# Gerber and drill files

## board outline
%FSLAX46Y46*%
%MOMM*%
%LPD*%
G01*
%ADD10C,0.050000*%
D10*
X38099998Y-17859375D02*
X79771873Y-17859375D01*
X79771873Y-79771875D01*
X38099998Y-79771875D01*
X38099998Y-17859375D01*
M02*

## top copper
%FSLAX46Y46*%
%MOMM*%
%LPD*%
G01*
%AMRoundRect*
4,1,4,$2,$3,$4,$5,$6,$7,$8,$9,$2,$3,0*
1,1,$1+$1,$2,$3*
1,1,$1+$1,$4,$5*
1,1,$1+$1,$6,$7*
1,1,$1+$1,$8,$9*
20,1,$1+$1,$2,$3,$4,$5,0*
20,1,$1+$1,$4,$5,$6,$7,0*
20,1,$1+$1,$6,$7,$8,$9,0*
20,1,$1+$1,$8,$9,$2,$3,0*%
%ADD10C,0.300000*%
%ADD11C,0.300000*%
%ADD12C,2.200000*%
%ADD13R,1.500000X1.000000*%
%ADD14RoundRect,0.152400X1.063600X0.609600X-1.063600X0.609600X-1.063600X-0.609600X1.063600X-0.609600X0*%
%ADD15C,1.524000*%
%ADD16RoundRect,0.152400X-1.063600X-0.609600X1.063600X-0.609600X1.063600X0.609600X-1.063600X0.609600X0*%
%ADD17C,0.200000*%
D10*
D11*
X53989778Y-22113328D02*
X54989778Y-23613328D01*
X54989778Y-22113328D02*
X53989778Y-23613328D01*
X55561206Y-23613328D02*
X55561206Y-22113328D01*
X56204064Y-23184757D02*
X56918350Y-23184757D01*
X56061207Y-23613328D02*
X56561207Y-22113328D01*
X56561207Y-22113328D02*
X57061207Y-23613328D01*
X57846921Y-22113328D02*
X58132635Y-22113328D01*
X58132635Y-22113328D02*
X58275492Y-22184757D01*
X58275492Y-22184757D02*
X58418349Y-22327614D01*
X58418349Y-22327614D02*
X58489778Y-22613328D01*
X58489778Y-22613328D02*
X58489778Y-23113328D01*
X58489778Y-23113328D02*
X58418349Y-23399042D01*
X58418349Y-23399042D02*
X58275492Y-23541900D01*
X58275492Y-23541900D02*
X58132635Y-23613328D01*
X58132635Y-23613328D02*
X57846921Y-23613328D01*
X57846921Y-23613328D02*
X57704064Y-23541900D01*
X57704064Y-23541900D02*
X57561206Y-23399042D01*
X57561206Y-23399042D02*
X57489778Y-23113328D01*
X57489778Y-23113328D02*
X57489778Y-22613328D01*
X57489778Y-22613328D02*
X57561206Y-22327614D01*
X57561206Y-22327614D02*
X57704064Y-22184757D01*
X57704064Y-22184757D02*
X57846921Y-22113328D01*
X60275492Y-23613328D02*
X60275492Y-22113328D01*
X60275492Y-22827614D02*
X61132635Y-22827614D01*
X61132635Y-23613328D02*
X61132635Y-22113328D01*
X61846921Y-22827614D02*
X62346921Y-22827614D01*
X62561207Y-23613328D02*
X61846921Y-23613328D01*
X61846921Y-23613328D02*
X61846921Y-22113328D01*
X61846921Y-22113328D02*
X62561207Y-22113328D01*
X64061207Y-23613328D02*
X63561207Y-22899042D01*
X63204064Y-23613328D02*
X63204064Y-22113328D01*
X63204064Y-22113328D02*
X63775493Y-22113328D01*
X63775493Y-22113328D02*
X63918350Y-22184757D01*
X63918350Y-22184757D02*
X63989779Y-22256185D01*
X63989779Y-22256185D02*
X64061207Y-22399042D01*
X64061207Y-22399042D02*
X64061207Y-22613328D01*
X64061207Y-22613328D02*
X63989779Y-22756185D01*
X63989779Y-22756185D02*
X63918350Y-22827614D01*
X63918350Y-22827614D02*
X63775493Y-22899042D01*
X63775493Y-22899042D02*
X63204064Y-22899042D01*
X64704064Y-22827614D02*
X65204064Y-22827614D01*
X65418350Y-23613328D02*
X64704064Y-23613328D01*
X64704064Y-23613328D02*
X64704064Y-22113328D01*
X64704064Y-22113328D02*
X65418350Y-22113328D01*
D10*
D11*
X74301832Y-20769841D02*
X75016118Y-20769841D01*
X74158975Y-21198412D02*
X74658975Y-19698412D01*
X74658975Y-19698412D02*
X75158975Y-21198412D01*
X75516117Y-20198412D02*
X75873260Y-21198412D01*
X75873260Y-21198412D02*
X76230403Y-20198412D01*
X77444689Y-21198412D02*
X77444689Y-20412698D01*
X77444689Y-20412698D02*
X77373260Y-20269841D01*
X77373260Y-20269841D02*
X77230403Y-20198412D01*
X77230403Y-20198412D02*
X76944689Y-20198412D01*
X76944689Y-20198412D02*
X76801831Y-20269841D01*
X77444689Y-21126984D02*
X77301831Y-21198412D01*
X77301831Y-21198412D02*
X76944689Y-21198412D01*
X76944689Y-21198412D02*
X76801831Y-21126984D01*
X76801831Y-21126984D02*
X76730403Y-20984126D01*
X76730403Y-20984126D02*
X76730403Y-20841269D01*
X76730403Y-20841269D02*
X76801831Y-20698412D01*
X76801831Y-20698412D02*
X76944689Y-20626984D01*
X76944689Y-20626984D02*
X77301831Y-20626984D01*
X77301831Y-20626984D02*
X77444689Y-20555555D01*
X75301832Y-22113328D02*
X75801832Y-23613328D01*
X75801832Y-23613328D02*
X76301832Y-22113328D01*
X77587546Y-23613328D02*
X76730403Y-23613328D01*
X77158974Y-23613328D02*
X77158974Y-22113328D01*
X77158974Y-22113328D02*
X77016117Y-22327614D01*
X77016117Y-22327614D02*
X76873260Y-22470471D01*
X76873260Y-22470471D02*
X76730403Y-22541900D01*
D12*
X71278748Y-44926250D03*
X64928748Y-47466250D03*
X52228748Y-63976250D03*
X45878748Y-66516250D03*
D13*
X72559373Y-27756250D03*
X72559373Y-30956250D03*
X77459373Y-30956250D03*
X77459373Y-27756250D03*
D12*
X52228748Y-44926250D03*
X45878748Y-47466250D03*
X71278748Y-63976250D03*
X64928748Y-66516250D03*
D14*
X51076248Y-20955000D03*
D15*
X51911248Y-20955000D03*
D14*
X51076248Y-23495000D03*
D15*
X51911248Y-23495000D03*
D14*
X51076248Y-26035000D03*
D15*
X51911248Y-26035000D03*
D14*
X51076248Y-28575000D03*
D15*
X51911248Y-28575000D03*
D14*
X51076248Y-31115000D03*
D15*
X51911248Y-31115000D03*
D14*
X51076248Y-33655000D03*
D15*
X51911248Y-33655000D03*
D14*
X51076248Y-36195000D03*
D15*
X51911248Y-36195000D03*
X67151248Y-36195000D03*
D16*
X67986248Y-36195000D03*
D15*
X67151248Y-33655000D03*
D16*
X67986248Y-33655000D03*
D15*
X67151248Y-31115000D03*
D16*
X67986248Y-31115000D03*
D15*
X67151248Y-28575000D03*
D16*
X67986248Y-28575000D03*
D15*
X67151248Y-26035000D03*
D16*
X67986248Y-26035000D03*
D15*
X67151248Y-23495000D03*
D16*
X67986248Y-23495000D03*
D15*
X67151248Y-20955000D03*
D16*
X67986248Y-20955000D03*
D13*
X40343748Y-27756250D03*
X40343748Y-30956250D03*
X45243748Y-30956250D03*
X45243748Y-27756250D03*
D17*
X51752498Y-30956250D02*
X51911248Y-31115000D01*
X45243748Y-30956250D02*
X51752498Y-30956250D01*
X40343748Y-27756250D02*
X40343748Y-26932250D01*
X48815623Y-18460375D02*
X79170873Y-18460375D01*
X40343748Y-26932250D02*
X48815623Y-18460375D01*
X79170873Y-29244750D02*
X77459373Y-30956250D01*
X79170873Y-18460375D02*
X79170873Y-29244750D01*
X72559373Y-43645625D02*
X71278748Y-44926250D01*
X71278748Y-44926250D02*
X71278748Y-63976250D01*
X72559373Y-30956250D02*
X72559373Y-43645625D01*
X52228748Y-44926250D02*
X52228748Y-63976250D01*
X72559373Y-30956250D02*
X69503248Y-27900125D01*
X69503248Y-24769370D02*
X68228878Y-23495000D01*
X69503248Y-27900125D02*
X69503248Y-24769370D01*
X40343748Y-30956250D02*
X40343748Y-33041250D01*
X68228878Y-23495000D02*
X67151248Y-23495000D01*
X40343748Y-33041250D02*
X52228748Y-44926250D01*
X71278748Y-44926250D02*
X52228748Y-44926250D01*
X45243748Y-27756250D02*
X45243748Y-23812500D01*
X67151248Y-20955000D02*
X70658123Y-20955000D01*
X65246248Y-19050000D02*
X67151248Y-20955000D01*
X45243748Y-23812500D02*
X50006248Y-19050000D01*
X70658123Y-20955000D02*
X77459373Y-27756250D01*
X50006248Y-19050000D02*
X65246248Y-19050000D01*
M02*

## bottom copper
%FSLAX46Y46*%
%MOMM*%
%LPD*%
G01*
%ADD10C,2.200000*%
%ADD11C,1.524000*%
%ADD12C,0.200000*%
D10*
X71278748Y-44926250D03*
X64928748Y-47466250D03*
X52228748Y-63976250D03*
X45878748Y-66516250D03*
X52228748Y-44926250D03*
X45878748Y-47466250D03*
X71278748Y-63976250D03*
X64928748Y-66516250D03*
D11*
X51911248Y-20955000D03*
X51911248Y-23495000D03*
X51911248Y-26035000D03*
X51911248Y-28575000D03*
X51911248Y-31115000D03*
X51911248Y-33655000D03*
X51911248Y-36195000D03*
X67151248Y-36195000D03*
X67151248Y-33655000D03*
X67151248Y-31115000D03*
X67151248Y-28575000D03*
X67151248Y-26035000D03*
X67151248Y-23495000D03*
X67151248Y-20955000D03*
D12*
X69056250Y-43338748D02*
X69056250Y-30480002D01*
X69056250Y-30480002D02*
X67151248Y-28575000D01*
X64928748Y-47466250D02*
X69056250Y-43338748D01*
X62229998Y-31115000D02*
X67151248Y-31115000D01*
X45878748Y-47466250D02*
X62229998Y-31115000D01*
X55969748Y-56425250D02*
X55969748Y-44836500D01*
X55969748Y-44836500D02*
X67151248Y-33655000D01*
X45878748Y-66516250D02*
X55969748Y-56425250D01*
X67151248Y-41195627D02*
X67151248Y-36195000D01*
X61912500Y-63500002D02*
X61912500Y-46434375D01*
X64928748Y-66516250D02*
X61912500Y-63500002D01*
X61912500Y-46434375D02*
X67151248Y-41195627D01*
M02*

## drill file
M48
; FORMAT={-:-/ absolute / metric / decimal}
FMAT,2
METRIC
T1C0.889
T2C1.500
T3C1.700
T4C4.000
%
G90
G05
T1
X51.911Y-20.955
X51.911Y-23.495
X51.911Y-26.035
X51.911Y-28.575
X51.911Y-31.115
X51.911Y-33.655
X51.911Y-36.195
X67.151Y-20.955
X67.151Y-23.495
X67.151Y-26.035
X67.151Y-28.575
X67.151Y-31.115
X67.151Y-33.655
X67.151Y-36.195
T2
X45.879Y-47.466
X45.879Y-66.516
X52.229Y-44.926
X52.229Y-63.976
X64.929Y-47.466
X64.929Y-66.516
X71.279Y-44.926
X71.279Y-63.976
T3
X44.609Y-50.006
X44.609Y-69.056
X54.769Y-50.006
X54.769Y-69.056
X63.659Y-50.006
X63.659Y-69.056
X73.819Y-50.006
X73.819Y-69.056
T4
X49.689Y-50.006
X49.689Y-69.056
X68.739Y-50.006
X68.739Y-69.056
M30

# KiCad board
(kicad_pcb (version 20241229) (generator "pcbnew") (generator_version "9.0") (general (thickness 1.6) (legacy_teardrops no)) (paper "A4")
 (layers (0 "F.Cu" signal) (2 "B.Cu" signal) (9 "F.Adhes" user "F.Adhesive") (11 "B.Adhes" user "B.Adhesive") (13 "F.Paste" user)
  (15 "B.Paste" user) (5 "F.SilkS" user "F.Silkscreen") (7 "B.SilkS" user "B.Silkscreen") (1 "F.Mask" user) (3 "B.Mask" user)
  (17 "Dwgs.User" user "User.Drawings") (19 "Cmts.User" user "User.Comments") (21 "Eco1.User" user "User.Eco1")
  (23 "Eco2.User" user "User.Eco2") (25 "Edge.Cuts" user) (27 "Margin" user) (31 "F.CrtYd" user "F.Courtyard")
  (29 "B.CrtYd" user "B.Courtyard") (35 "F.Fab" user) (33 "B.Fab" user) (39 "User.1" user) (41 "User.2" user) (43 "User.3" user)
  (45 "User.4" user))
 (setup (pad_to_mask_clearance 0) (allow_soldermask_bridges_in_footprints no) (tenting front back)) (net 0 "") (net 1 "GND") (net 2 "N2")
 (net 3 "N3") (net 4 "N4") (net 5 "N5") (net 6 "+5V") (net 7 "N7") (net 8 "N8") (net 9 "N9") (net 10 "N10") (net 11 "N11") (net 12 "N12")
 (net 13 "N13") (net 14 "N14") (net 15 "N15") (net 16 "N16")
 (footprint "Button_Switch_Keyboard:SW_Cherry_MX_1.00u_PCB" (layer "F.Cu") (at 71.278748 44.92625)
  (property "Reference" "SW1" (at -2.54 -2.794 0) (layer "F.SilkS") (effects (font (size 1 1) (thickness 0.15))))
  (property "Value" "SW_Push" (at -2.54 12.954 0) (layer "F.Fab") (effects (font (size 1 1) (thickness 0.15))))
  (pad "" np_thru_hole circle (at -7.62 5.08) (size 1.7 1.7) (drill 1.7) (layers "*.Cu" "*.Mask"))
  (pad "" np_thru_hole circle (at -2.54 5.08) (size 4 4) (drill 4) (layers "*.Cu" "*.Mask"))
  (pad "" np_thru_hole circle (at 2.54 5.08) (size 1.7 1.7) (drill 1.7) (layers "*.Cu" "*.Mask"))
  (pad "1" thru_hole circle (at 0 0) (size 2.2 2.2) (drill 1.5) (layers "*.Cu" "*.Mask") (remove_unused_layers no) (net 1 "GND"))
  (pad "2" thru_hole circle (at -6.35 2.54) (size 2.2 2.2) (drill 1.5) (layers "*.Cu" "*.Mask") (remove_unused_layers no) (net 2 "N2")))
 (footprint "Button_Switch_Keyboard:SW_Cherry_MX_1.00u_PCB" (layer "F.Cu") (at 52.228748 63.97625)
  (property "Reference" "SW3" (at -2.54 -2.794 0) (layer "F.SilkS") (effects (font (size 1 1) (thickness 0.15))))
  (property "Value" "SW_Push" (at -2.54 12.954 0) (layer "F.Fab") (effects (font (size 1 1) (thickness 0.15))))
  (pad "" np_thru_hole circle (at -7.62 5.08) (size 1.7 1.7) (drill 1.7) (layers "*.Cu" "*.Mask"))
  (pad "" np_thru_hole circle (at -2.54 5.08) (size 4 4) (drill 4) (layers "*.Cu" "*.Mask"))
  (pad "" np_thru_hole circle (at 2.54 5.08) (size 1.7 1.7) (drill 1.7) (layers "*.Cu" "*.Mask"))
  (pad "1" thru_hole circle (at 0 0) (size 2.2 2.2) (drill 1.5) (layers "*.Cu" "*.Mask") (remove_unused_layers no) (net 1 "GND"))
  (pad "2" thru_hole circle (at -6.35 2.54) (size 2.2 2.2) (drill 1.5) (layers "*.Cu" "*.Mask") (remove_unused_layers no) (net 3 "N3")))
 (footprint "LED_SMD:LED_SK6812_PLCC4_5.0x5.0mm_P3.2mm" (layer "F.Cu") (at 75.009373 29.35625)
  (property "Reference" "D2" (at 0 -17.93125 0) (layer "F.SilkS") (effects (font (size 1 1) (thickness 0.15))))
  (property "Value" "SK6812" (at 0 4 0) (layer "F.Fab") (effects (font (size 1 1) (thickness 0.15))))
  (pad "1" smd rect (at -2.45 -1.6 180) (size 1.5 1) (layers "F.Cu" "F.Mask" "F.Paste") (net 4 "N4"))
  (pad "2" smd rect (at -2.45 1.6 180) (size 1.5 1) (layers "F.Cu" "F.Mask" "F.Paste") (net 1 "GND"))
  (pad "3" smd rect (at 2.45 1.6 180) (size 1.5 1) (layers "F.Cu" "F.Mask" "F.Paste") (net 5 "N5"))
  (pad "4" smd rect (at 2.45 -1.6 180) (size 1.5 1) (layers "F.Cu" "F.Mask" "F.Paste") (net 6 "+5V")))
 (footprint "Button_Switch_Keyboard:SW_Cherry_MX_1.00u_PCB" (layer "F.Cu") (at 52.228748 44.92625)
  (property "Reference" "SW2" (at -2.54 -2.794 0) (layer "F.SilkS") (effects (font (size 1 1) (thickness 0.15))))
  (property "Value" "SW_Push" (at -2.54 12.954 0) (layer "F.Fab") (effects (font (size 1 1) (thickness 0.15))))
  (pad "" np_thru_hole circle (at -7.62 5.08) (size 1.7 1.7) (drill 1.7) (layers "*.Cu" "*.Mask"))
  (pad "" np_thru_hole circle (at -2.54 5.08) (size 4 4) (drill 4) (layers "*.Cu" "*.Mask"))
  (pad "" np_thru_hole circle (at 2.54 5.08) (size 1.7 1.7) (drill 1.7) (layers "*.Cu" "*.Mask"))
  (pad "1" thru_hole circle (at 0 0) (size 2.2 2.2) (drill 1.5) (layers "*.Cu" "*.Mask") (remove_unused_layers no) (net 1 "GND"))
  (pad "2" thru_hole circle (at -6.35 2.54) (size 2.2 2.2) (drill 1.5) (layers "*.Cu" "*.Mask") (remove_unused_layers no) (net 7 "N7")))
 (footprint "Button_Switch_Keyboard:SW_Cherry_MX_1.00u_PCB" (layer "F.Cu") (at 71.278748 63.97625)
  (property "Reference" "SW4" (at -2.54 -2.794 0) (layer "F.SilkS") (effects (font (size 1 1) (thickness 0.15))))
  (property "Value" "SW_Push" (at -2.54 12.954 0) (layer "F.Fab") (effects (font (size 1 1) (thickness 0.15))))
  (pad "" np_thru_hole circle (at -7.62 5.08) (size 1.7 1.7) (drill 1.7) (layers "*.Cu" "*.Mask"))
  (pad "" np_thru_hole circle (at -2.54 5.08) (size 4 4) (drill 4) (layers "*.Cu" "*.Mask"))
  (pad "" np_thru_hole circle (at 2.54 5.08) (size 1.7 1.7) (drill 1.7) (layers "*.Cu" "*.Mask"))
  (pad "1" thru_hole circle (at 0 0) (size 2.2 2.2) (drill 1.5) (layers "*.Cu" "*.Mask") (remove_unused_layers no) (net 1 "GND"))
  (pad "2" thru_hole circle (at -6.35 2.54) (size 2.2 2.2) (drill 1.5) (layers "*.Cu" "*.Mask") (remove_unused_layers no) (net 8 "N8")))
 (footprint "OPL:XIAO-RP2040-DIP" (layer "F.Cu") (at 59.531248 28.575)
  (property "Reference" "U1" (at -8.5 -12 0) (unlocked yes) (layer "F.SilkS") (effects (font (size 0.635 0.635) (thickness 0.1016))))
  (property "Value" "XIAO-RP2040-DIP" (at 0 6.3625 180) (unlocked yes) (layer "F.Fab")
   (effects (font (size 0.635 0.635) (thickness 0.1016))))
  (pad "1" smd roundrect (at -8.455 -7.62 180) (size 2.432 1.524) (layers "F.Cu" "F.Mask") (roundrect_rratio 0.1) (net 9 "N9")
   (thermal_bridge_angle 45))
  (pad "1" thru_hole circle (at -7.62 -7.62 180) (size 1.524 1.524) (drill 0.889) (layers "*.Cu" "*.Mask") (remove_unused_layers no)
   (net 9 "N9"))
  (pad "2" smd roundrect (at -8.455 -5.08 180) (size 2.432 1.524) (layers "F.Cu" "F.Mask") (roundrect_rratio 0.1) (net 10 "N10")
   (thermal_bridge_angle 45))
  (pad "2" thru_hole circle (at -7.62 -5.08 180) (size 1.524 1.524) (drill 0.889) (layers "*.Cu" "*.Mask") (remove_unused_layers no)
   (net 10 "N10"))
  (pad "3" smd roundrect (at -8.455 -2.54 180) (size 2.432 1.524) (layers "F.Cu" "F.Mask") (roundrect_rratio 0.1) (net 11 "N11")
   (thermal_bridge_angle 45))
  (pad "3" thru_hole circle (at -7.62 -2.54 180) (size 1.524 1.524) (drill 0.889) (layers "*.Cu" "*.Mask") (remove_unused_layers no)
   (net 11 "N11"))
  (pad "4" smd roundrect (at -8.455 0 180) (size 2.432 1.524) (layers "F.Cu" "F.Mask") (roundrect_rratio 0.1) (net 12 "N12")
   (thermal_bridge_angle 45))
  (pad "4" thru_hole circle (at -7.62 0 180) (size 1.524 1.524) (drill 0.889) (layers "*.Cu" "*.Mask") (remove_unused_layers no)
   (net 12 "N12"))
  (pad "5" smd roundrect (at -8.455 2.54 180) (size 2.432 1.524) (layers "F.Cu" "F.Mask") (roundrect_rratio 0.1) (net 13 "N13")
   (thermal_bridge_angle 45))
  (pad "5" thru_hole circle (at -7.62 2.54 180) (size 1.524 1.524) (drill 0.889) (layers "*.Cu" "*.Mask") (remove_unused_layers no)
   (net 13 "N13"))
  (pad "6" smd roundrect (at -8.455 5.08 180) (size 2.432 1.524) (layers "F.Cu" "F.Mask") (roundrect_rratio 0.1) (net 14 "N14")
   (thermal_bridge_angle 45))
  (pad "6" thru_hole circle (at -7.62 5.08 180) (size 1.524 1.524) (drill 0.889) (layers "*.Cu" "*.Mask") (remove_unused_layers no)
   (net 14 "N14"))
  (pad "7" smd roundrect (at -8.455 7.62 180) (size 2.432 1.524) (layers "F.Cu" "F.Mask") (roundrect_rratio 0.1) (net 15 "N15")
   (thermal_bridge_angle 45))
  (pad "7" thru_hole circle (at -7.62 7.62 180) (size 1.524 1.524) (drill 0.889) (layers "*.Cu" "*.Mask") (remove_unused_layers no)
   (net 15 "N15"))
  (pad "8" thru_hole circle (at 7.62 7.62) (size 1.524 1.524) (drill 0.889) (layers "*.Cu" "*.Mask") (remove_unused_layers no) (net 8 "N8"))
  (pad "8" smd roundrect (at 8.455 7.62) (size 2.432 1.524) (layers "F.Cu" "F.Mask") (roundrect_rratio 0.1) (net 8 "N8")
   (thermal_bridge_angle 45))
  (pad "9" thru_hole circle (at 7.62 5.08) (size 1.524 1.524) (drill 0.889) (layers "*.Cu" "*.Mask") (remove_unused_layers no) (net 3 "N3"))
  (pad "9" smd roundrect (at 8.455 5.08) (size 2.432 1.524) (layers "F.Cu" "F.Mask") (roundrect_rratio 0.1) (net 3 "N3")
   (thermal_bridge_angle 45))
  (pad "10" thru_hole circle (at 7.62 2.54) (size 1.524 1.524) (drill 0.889) (layers "*.Cu" "*.Mask") (remove_unused_layers no) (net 7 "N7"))
  (pad "10" smd roundrect (at 8.455 2.54) (size 2.432 1.524) (layers "F.Cu" "F.Mask") (roundrect_rratio 0.1) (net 7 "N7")
   (thermal_bridge_angle 45))
  (pad "11" thru_hole circle (at 7.62 0) (size 1.524 1.524) (drill 0.889) (layers "*.Cu" "*.Mask") (remove_unused_layers no) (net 2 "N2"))
  (pad "11" smd roundrect (at 8.455 0) (size 2.432 1.524) (layers "F.Cu" "F.Mask") (roundrect_rratio 0.1) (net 2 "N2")
   (thermal_bridge_angle 45))
  (pad "12" thru_hole circle (at 7.62 -2.54) (size 1.524 1.524) (drill 0.889) (layers "*.Cu" "*.Mask") (remove_unused_layers no)
   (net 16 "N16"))
  (pad "12" smd roundrect (at 8.455 -2.54) (size 2.432 1.524) (layers "F.Cu" "F.Mask") (roundrect_rratio 0.1) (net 16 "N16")
   (thermal_bridge_angle 45))
  (pad "13" thru_hole circle (at 7.62 -5.08) (size 1.524 1.524) (drill 0.889) (layers "*.Cu" "*.Mask") (remove_unused_layers no)
   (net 1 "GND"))
  (pad "13" smd roundrect (at 8.455 -5.08) (size 2.432 1.524) (layers "F.Cu" "F.Mask") (roundrect_rratio 0.1) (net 1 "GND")
   (thermal_bridge_angle 45))
  (pad "14" thru_hole circle (at 7.62 -7.62) (size 1.524 1.524) (drill 0.889) (layers "*.Cu" "*.Mask") (remove_unused_layers no)
   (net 6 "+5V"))
  (pad "14" smd roundrect (at 8.455 -7.62) (size 2.432 1.524) (layers "F.Cu" "F.Mask") (roundrect_rratio 0.1) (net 6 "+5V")
   (thermal_bridge_angle 45)))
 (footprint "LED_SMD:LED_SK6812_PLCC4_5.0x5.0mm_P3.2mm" (layer "F.Cu") (at 42.793748 29.35625)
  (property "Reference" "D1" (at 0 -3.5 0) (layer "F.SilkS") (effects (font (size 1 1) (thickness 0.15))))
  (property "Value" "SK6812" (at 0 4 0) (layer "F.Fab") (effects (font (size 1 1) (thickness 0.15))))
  (pad "1" smd rect (at -2.45 -1.6 180) (size 1.5 1) (layers "F.Cu" "F.Mask" "F.Paste") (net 5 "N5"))
  (pad "2" smd rect (at -2.45 1.6 180) (size 1.5 1) (layers "F.Cu" "F.Mask" "F.Paste") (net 1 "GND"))
  (pad "3" smd rect (at 2.45 1.6 180) (size 1.5 1) (layers "F.Cu" "F.Mask" "F.Paste") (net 13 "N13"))
  (pad "4" smd rect (at 2.45 -1.6 180) (size 1.5 1) (layers "F.Cu" "F.Mask" "F.Paste") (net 6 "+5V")))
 (gr_rect (start 38.099998 17.859375) (end 79.771873 79.771875) (stroke (width 0.05) (type default)) (fill no) (layer "Edge.Cuts"))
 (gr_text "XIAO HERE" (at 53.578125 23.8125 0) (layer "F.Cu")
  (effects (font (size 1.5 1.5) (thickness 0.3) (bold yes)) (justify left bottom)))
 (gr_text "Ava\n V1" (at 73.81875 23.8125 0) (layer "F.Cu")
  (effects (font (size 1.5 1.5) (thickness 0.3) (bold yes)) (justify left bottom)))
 (segment (start 51.752498 30.95625) (end 51.911248 31.115) (width 0.2) (layer "F.Cu") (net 13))
 (segment (start 45.243748 30.95625) (end 51.752498 30.95625) (width 0.2) (layer "F.Cu") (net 13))
 (segment (start 40.343748 27.75625) (end 40.343748 26.93225) (width 0.2) (layer "F.Cu") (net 5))
 (segment (start 48.815623 18.460375) (end 79.170873 18.460375) (width 0.2) (layer "F.Cu") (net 5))
 (segment (start 40.343748 26.93225) (end 48.815623 18.460375) (width 0.2) (layer "F.Cu") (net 5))
 (segment (start 79.170873 29.24475) (end 77.459373 30.95625) (width 0.2) (layer "F.Cu") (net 5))
 (segment (start 79.170873 18.460375) (end 79.170873 29.24475) (width 0.2) (layer "F.Cu") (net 5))
 (segment (start 72.559373 43.645625) (end 71.278748 44.92625) (width 0.2) (layer "F.Cu") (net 1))
 (segment (start 71.278748 44.92625) (end 71.278748 63.97625) (width 0.2) (layer "F.Cu") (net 1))
 (segment (start 72.559373 30.95625) (end 72.559373 43.645625) (width 0.2) (layer "F.Cu") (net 1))
 (segment (start 52.228748 44.92625) (end 52.228748 63.97625) (width 0.2) (layer "F.Cu") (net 1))
 (segment (start 72.559373 30.95625) (end 69.503248 27.900125) (width 0.2) (layer "F.Cu") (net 1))
 (segment (start 69.503248 24.76937) (end 68.228878 23.495) (width 0.2) (layer "F.Cu") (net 1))
 (segment (start 69.503248 27.900125) (end 69.503248 24.76937) (width 0.2) (layer "F.Cu") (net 1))
 (segment (start 40.343748 30.95625) (end 40.343748 33.04125) (width 0.2) (layer "F.Cu") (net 1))
 (segment (start 68.228878 23.495) (end 67.151248 23.495) (width 0.2) (layer "F.Cu") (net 1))
 (segment (start 40.343748 33.04125) (end 52.228748 44.92625) (width 0.2) (layer "F.Cu") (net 1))
 (segment (start 71.278748 44.92625) (end 52.228748 44.92625) (width 0.2) (layer "F.Cu") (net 1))
 (segment (start 69.05625 43.338748) (end 69.05625 30.480002) (width 0.2) (layer "B.Cu") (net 2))
 (segment (start 69.05625 30.480002) (end 67.151248 28.575) (width 0.2) (layer "B.Cu") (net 2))
 (segment (start 64.928748 47.46625) (end 69.05625 43.338748) (width 0.2) (layer "B.Cu") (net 2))
 (segment (start 62.229998 31.115) (end 67.151248 31.115) (width 0.2) (layer "B.Cu") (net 7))
 (segment (start 45.878748 47.46625) (end 62.229998 31.115) (width 0.2) (layer "B.Cu") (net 7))
 (segment (start 55.969748 56.42525) (end 55.969748 44.8365) (width 0.2) (layer "B.Cu") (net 3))
 (segment (start 55.969748 44.8365) (end 67.151248 33.655) (width 0.2) (layer "B.Cu") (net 3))
 (segment (start 45.878748 66.51625) (end 55.969748 56.42525) (width 0.2) (layer "B.Cu") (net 3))
 (segment (start 67.151248 41.195627) (end 67.151248 36.195) (width 0.2) (layer "B.Cu") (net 8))
 (segment (start 61.9125 63.500002) (end 61.9125 46.434375) (width 0.2) (layer "B.Cu") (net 8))
 (segment (start 64.928748 66.51625) (end 61.9125 63.500002) (width 0.2) (layer "B.Cu") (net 8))
 (segment (start 61.9125 46.434375) (end 67.151248 41.195627) (width 0.2) (layer "B.Cu") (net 8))
 (segment (start 45.243748 27.75625) (end 45.243748 23.8125) (width 0.2) (layer "F.Cu") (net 6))
 (segment (start 67.151248 20.955) (end 70.658123 20.955) (width 0.2) (layer "F.Cu") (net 6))
 (segment (start 65.246248 19.05) (end 67.151248 20.955) (width 0.2) (layer "F.Cu") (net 6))
 (segment (start 45.243748 23.8125) (end 50.006248 19.05) (width 0.2) (layer "F.Cu") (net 6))
 (segment (start 70.658123 20.955) (end 77.459373 27.75625) (width 0.2) (layer "F.Cu") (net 6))
 (segment (start 50.006248 19.05) (end 65.246248 19.05) (width 0.2) (layer "F.Cu") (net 6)))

